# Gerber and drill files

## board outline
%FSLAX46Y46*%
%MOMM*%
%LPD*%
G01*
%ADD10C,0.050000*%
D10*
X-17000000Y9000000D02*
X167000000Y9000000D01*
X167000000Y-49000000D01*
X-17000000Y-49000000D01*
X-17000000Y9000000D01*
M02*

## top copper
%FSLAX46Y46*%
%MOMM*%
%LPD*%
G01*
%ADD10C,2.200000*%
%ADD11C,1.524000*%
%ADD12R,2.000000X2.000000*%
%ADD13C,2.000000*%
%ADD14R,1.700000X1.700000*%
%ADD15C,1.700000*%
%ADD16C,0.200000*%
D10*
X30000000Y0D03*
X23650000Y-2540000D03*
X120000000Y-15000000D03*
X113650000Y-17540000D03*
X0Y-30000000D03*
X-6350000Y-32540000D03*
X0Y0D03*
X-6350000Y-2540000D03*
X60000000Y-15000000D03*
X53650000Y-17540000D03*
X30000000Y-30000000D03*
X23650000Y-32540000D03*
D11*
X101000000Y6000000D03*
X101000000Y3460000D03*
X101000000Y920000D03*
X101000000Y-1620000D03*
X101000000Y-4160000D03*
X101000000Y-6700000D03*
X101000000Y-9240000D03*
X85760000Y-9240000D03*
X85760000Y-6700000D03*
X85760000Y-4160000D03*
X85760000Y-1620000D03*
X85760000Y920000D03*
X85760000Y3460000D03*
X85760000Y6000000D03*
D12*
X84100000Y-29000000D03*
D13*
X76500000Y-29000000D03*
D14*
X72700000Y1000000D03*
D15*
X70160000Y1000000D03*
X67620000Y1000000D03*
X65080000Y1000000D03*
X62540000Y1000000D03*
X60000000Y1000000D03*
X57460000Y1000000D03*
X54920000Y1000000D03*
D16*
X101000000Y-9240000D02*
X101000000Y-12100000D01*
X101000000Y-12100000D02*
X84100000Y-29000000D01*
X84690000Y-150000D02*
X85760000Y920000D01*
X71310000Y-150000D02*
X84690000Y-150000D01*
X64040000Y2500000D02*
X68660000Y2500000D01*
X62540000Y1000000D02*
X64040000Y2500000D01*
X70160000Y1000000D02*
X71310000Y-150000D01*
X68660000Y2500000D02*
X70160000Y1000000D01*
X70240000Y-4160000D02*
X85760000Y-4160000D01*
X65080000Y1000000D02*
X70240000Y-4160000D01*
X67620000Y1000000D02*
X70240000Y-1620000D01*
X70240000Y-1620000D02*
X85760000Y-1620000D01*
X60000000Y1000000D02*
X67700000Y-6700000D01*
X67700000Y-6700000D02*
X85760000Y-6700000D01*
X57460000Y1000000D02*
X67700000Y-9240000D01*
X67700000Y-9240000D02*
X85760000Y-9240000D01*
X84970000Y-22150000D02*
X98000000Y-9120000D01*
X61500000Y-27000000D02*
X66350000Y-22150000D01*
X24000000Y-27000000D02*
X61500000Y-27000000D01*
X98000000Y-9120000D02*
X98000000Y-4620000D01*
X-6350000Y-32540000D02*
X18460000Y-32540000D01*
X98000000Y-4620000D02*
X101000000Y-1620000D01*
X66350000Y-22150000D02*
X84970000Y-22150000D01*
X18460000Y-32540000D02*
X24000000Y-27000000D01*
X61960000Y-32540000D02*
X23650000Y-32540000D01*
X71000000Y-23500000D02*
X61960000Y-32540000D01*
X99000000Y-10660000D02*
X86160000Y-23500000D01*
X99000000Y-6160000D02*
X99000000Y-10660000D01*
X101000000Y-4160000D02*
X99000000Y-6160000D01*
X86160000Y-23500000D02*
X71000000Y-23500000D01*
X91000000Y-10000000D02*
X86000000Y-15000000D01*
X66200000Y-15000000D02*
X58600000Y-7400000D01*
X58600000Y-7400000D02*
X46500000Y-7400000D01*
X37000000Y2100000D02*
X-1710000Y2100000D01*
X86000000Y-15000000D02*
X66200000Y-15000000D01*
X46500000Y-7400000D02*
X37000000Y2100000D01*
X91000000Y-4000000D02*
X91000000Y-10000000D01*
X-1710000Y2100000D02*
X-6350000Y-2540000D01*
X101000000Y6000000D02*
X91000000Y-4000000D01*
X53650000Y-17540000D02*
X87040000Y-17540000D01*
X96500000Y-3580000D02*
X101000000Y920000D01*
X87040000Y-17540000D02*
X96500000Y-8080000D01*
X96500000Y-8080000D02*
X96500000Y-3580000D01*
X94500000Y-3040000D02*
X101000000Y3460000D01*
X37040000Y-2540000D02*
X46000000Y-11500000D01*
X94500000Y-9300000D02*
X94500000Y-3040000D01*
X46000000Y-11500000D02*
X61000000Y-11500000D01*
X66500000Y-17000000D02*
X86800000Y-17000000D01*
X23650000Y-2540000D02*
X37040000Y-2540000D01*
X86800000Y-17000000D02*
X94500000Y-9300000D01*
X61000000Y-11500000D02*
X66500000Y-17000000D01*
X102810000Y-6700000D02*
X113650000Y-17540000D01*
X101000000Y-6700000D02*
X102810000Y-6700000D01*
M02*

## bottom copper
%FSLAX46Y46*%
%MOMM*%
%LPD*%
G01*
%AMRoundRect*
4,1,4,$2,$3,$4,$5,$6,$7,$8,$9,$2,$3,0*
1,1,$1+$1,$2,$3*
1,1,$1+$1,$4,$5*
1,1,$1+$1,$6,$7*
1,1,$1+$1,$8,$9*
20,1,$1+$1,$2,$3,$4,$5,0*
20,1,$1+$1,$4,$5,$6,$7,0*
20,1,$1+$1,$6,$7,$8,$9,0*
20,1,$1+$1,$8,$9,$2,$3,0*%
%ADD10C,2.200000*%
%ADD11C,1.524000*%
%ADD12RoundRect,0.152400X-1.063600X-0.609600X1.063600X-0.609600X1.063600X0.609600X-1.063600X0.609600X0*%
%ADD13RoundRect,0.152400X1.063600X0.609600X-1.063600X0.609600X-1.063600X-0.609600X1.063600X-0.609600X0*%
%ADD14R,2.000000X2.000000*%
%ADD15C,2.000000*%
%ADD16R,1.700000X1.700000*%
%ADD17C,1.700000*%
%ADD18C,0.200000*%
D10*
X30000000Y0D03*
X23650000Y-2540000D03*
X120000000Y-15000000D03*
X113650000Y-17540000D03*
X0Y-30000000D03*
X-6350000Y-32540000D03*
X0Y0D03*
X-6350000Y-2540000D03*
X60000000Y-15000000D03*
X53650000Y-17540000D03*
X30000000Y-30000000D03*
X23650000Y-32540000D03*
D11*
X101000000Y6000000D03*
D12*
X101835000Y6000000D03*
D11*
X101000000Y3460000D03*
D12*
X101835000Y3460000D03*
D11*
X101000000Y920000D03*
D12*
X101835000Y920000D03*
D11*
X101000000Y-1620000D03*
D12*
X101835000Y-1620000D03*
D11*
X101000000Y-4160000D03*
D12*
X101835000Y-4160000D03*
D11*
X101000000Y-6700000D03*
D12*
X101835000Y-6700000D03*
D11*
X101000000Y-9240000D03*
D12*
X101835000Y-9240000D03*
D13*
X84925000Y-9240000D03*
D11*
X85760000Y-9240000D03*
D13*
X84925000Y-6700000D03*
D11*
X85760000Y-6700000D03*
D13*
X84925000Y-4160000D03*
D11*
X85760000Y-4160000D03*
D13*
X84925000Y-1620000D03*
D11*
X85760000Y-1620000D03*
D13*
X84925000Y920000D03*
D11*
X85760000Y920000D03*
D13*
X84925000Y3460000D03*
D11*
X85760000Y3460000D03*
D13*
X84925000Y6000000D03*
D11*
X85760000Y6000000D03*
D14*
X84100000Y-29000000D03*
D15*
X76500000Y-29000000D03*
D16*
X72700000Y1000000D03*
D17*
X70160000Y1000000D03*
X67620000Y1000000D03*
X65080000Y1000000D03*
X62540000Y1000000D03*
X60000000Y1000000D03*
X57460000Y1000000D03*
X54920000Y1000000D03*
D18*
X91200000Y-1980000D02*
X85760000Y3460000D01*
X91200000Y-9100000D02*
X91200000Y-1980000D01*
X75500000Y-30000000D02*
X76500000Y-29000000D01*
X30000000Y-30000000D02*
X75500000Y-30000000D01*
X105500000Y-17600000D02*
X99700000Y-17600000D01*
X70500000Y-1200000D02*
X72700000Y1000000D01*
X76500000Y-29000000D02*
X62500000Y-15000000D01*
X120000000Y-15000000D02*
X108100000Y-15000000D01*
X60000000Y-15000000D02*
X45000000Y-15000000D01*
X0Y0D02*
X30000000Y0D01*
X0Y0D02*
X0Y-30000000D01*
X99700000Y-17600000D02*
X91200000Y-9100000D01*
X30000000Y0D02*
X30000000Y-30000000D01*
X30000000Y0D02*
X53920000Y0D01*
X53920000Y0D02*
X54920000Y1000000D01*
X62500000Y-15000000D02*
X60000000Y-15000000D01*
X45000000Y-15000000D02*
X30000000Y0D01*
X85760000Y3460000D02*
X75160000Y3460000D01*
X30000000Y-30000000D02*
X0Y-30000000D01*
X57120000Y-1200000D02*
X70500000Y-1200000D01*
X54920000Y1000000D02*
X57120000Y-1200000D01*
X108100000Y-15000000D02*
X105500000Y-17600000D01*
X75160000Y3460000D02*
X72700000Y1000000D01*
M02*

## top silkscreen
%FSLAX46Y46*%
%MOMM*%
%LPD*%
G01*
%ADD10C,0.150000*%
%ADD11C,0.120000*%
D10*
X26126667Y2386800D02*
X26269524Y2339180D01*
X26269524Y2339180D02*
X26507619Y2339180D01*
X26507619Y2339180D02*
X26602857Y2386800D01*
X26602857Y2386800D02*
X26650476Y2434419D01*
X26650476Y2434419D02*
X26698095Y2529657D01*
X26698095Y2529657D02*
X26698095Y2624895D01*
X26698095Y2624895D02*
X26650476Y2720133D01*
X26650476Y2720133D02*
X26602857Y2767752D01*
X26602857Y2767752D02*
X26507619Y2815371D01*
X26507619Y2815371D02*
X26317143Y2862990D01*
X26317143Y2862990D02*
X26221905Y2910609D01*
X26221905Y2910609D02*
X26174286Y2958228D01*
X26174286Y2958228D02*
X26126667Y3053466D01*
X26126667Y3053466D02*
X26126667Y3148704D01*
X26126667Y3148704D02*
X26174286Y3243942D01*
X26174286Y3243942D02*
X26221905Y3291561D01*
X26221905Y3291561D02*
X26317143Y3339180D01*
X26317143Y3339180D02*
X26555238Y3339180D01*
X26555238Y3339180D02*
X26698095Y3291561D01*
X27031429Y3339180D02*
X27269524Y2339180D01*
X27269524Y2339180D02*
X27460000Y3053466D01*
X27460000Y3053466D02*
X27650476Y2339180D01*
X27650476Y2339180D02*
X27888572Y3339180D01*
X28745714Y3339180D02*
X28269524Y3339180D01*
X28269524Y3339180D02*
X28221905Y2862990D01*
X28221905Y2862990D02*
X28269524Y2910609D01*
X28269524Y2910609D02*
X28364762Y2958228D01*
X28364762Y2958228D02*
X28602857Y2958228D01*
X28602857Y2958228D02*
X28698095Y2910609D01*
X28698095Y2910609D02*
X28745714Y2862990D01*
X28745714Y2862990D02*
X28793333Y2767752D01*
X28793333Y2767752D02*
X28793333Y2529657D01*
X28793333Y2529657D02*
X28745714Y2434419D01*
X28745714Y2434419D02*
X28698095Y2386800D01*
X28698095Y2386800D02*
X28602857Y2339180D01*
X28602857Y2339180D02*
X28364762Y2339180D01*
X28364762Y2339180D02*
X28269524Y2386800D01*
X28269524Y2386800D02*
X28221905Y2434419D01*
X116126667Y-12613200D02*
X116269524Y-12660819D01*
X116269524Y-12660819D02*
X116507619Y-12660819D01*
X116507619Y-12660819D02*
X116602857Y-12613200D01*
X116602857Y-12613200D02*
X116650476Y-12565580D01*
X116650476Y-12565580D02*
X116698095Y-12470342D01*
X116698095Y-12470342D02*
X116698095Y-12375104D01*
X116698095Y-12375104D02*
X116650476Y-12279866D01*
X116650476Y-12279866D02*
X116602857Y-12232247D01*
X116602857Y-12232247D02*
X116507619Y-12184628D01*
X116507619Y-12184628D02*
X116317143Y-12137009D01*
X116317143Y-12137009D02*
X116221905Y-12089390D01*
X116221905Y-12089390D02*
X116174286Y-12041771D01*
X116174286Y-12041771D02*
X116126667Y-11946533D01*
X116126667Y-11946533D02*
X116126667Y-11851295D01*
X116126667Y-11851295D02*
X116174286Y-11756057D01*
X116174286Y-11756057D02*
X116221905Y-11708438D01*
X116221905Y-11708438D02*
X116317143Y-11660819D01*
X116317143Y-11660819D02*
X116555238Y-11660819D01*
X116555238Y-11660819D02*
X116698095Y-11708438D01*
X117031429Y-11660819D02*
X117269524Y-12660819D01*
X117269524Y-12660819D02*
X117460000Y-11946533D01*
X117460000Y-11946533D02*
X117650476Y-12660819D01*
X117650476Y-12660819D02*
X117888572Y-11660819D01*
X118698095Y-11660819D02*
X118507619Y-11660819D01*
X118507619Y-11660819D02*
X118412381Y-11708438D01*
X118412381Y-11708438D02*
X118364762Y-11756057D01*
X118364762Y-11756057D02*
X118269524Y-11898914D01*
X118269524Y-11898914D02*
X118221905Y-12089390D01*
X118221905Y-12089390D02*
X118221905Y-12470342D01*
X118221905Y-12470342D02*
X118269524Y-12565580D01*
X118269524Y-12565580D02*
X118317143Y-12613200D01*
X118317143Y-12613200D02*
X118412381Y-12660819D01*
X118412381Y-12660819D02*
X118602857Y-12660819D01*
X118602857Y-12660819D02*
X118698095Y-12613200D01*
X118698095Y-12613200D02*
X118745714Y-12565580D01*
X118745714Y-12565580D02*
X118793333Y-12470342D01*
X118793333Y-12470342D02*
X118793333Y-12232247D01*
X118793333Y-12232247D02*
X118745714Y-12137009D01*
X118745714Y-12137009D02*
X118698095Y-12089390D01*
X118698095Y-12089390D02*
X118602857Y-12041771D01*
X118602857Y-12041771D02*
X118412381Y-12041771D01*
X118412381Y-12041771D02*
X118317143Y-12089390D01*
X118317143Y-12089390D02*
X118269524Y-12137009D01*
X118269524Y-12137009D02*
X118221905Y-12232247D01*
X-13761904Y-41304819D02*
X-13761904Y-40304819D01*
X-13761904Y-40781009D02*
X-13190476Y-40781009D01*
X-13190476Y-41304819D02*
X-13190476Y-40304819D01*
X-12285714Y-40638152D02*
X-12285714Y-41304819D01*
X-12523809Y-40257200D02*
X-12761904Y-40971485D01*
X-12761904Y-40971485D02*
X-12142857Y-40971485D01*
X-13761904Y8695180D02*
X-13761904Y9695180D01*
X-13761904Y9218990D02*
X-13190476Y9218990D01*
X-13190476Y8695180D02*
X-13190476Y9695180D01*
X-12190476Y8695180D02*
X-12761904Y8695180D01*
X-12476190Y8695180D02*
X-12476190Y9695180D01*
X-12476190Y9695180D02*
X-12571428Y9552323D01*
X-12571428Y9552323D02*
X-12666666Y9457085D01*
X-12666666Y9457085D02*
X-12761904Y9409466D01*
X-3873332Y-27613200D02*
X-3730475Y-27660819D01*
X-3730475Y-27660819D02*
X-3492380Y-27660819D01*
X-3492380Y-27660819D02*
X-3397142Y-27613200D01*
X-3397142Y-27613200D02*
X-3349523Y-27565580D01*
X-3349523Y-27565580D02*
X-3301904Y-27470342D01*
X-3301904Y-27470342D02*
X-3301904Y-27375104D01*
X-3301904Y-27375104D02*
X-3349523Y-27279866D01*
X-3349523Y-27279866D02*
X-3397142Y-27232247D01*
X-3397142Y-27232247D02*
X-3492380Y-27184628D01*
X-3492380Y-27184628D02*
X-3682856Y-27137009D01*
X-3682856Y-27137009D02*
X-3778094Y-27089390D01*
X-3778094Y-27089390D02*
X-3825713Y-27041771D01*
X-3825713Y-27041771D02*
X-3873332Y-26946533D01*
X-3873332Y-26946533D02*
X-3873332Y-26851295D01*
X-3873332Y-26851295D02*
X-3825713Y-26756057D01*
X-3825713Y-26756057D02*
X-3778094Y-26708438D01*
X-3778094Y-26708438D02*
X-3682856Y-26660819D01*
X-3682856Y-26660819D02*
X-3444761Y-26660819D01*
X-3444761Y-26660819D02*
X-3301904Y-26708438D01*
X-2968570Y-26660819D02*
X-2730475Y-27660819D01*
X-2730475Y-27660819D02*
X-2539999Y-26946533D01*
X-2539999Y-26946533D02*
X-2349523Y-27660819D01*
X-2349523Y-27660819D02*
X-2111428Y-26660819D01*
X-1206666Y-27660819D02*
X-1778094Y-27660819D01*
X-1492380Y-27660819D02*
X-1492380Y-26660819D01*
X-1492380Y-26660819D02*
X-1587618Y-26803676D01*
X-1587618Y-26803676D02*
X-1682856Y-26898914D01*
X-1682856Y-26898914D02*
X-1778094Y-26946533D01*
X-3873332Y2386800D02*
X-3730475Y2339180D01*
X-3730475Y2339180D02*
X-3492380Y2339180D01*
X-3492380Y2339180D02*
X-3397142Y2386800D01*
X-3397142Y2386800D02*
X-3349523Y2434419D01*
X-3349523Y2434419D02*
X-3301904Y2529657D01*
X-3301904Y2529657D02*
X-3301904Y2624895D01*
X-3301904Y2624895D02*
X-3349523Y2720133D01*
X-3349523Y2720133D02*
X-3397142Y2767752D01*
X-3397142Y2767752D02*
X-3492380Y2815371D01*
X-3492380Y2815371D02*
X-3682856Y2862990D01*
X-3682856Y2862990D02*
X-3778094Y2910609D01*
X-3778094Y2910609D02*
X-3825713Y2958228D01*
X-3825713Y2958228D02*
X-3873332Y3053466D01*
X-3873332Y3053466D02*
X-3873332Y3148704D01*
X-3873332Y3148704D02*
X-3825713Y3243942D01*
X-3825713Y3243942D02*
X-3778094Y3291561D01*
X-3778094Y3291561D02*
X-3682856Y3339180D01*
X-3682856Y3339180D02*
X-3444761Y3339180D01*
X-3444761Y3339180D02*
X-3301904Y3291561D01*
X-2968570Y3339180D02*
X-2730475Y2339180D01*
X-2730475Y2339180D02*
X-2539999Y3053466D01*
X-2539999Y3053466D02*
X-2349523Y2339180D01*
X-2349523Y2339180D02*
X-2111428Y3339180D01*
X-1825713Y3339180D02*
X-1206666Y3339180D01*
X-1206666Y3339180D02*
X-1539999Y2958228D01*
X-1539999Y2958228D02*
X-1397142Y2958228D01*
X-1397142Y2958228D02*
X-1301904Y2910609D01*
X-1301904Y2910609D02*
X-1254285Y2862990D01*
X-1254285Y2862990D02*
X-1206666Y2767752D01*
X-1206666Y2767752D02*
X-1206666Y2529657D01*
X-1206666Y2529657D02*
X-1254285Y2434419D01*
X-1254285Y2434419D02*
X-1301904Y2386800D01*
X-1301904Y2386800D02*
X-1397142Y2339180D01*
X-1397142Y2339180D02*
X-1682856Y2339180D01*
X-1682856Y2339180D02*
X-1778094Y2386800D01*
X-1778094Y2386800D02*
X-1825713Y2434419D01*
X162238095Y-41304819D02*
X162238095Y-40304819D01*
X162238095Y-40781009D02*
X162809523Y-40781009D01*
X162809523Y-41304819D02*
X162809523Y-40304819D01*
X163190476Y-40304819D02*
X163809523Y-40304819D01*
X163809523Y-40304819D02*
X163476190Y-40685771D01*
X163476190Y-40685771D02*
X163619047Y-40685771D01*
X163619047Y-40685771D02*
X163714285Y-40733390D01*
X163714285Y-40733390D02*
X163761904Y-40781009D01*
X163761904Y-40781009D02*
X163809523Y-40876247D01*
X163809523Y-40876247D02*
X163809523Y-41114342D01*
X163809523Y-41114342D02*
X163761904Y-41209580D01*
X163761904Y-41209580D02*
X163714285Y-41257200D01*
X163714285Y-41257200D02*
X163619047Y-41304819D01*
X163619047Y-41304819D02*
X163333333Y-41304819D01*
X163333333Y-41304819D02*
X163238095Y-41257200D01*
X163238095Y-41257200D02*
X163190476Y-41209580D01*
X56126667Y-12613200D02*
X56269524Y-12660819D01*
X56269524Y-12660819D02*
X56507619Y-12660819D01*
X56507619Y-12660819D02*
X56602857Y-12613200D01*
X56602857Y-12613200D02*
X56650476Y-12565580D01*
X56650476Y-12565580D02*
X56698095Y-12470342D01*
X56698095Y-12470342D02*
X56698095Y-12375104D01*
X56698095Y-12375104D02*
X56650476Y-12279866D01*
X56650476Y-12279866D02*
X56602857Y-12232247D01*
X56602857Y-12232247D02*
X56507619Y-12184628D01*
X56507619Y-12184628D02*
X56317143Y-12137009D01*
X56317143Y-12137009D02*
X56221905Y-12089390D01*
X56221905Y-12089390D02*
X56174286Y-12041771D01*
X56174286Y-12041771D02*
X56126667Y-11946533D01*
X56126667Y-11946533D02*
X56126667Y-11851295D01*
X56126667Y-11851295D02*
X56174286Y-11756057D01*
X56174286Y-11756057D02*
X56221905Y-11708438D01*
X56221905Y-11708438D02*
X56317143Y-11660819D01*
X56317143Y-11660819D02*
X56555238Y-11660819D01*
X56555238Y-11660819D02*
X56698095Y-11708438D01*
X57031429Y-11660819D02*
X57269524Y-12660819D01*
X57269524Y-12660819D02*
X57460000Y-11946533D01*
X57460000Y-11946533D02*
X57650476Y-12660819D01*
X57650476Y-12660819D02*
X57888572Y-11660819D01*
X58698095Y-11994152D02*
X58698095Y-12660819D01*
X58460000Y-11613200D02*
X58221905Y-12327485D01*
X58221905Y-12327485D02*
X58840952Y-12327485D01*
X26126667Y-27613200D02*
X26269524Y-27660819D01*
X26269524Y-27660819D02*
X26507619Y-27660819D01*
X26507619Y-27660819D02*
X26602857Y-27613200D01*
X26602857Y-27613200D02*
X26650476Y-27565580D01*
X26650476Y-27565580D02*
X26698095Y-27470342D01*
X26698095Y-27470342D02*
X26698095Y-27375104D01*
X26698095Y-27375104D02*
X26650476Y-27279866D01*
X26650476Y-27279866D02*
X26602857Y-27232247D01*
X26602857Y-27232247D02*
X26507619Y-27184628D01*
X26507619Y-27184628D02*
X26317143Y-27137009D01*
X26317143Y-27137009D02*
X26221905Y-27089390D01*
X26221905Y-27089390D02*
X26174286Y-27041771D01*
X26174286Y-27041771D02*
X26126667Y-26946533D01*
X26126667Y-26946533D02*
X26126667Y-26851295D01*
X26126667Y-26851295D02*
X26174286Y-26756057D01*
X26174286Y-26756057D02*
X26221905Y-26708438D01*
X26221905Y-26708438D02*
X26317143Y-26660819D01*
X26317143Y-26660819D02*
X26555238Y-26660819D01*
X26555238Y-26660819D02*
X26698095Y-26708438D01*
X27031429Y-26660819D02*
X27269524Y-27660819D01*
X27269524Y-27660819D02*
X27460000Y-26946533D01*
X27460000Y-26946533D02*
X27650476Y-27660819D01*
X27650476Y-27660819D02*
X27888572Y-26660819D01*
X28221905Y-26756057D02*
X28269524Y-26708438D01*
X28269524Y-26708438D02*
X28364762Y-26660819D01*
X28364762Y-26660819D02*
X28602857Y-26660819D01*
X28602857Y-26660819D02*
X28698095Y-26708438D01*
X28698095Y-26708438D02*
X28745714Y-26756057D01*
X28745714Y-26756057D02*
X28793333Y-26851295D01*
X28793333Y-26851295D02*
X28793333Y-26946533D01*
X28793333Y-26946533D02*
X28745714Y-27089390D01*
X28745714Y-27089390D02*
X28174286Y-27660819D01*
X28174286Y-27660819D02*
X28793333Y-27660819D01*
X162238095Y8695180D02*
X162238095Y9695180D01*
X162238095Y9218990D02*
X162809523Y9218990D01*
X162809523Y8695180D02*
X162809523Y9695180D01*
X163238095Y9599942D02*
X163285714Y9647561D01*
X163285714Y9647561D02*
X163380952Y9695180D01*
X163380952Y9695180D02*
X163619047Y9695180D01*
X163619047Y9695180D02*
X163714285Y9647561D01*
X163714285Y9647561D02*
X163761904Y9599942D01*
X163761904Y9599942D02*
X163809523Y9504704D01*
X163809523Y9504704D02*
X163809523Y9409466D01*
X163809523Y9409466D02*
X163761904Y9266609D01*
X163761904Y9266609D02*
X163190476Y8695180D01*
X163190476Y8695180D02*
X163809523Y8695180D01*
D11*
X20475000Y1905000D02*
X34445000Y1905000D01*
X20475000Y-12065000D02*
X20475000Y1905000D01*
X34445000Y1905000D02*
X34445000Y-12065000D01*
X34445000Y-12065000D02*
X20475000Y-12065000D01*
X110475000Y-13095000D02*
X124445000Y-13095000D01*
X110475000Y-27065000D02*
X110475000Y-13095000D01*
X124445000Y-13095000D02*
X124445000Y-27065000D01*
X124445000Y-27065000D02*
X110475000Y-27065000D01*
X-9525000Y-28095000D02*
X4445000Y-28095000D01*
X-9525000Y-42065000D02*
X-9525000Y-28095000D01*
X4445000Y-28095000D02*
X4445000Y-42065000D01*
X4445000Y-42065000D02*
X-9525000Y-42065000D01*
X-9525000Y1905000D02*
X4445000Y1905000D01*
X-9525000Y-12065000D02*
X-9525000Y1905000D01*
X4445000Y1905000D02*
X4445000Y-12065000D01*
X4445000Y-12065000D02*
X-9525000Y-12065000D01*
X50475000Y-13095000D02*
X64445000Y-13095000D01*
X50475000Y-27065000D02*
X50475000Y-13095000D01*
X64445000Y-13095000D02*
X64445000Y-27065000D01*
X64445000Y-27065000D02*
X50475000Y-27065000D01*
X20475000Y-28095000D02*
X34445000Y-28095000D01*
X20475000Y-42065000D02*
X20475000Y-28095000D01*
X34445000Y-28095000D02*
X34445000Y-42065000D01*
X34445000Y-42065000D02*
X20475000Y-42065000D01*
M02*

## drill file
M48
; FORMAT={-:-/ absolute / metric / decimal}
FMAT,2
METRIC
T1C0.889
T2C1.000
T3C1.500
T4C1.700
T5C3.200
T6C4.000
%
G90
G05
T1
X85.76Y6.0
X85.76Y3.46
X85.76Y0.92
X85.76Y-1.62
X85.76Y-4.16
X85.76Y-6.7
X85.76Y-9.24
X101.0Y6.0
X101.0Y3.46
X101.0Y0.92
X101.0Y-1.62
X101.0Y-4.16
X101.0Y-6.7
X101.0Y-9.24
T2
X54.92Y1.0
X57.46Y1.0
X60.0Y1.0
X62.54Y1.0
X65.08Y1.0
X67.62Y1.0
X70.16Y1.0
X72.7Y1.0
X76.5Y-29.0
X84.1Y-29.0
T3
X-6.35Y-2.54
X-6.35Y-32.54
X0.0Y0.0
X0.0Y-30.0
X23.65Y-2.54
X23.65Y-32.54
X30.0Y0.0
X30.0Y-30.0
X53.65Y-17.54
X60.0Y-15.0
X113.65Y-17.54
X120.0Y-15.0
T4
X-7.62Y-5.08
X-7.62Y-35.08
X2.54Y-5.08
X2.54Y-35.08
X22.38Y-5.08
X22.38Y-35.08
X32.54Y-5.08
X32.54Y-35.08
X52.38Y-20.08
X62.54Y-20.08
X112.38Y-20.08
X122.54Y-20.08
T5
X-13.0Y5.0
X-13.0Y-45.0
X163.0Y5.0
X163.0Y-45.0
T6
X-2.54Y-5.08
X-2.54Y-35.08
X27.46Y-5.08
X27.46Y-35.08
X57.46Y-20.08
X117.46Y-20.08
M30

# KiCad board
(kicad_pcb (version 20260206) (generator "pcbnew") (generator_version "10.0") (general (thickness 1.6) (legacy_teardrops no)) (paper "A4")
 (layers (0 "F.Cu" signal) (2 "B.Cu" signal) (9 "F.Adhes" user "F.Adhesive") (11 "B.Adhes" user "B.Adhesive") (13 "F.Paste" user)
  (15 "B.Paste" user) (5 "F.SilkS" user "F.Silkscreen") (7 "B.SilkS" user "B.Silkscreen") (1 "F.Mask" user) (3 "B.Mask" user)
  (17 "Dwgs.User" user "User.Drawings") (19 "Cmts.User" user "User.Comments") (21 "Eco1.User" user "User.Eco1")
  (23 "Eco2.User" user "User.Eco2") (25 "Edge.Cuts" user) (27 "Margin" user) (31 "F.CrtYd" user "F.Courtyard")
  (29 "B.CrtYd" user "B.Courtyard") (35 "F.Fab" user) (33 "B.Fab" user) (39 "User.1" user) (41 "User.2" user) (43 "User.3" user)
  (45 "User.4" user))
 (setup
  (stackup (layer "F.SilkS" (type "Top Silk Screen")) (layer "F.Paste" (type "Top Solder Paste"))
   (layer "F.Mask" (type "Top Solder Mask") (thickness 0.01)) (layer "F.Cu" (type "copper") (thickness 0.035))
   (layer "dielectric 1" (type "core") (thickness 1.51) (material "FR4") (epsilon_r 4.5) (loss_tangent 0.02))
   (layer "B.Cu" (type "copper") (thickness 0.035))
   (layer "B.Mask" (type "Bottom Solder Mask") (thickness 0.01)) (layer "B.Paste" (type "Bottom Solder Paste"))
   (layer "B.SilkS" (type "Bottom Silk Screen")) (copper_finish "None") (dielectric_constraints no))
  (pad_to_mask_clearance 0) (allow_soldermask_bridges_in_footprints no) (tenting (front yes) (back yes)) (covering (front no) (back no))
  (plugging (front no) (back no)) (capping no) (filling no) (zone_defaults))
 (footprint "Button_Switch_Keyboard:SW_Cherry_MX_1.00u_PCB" (layer "F.Cu") (at 30 0)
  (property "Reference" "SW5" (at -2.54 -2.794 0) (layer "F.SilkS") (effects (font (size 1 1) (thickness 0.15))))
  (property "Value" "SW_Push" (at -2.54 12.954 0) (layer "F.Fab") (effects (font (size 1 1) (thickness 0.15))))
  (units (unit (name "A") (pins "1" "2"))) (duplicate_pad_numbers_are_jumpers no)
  (fp_line (start -9.525 -1.905) (end 4.445 -1.905) (stroke (width 0.12) (type solid)) (layer "F.SilkS"))
  (fp_line (start -9.525 12.065) (end -9.525 -1.905) (stroke (width 0.12) (type solid)) (layer "F.SilkS"))
  (fp_line (start 4.445 -1.905) (end 4.445 12.065) (stroke (width 0.12) (type solid)) (layer "F.SilkS"))
  (fp_line (start 4.445 12.065) (end -9.525 12.065) (stroke (width 0.12) (type solid)) (layer "F.SilkS"))
  (pad "" np_thru_hole circle (at -7.62 5.08) (size 1.7 1.7) (drill 1.7) (layers "*.Cu" "*.Mask"))
  (pad "" np_thru_hole circle (at -2.54 5.08) (size 4 4) (drill 4) (layers "*.Cu" "*.Mask"))
  (pad "" np_thru_hole circle (at 2.54 5.08) (size 1.7 1.7) (drill 1.7) (layers "*.Cu" "*.Mask"))
  (pad "1" thru_hole circle (at 0 0) (size 2.2 2.2) (drill 1.5) (layers "*.Cu" "*.Mask") (remove_unused_layers no) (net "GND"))
  (pad "2" thru_hole circle (at -6.35 2.54) (size 2.2 2.2) (drill 1.5) (layers "*.Cu" "*.Mask") (remove_unused_layers no) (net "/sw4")))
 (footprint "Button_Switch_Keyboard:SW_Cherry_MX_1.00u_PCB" (layer "F.Cu") (at 120 15)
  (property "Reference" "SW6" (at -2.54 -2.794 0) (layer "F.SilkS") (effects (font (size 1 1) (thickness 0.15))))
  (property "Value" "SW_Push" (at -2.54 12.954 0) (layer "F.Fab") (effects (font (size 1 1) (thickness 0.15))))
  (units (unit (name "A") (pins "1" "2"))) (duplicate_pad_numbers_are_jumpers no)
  (fp_line (start -9.525 -1.905) (end 4.445 -1.905) (stroke (width 0.12) (type solid)) (layer "F.SilkS"))
  (fp_line (start -9.525 12.065) (end -9.525 -1.905) (stroke (width 0.12) (type solid)) (layer "F.SilkS"))
  (fp_line (start 4.445 -1.905) (end 4.445 12.065) (stroke (width 0.12) (type solid)) (layer "F.SilkS"))
  (fp_line (start 4.445 12.065) (end -9.525 12.065) (stroke (width 0.12) (type solid)) (layer "F.SilkS"))
  (pad "" np_thru_hole circle (at -7.62 5.08) (size 1.7 1.7) (drill 1.7) (layers "*.Cu" "*.Mask"))
  (pad "" np_thru_hole circle (at -2.54 5.08) (size 4 4) (drill 4) (layers "*.Cu" "*.Mask"))
  (pad "" np_thru_hole circle (at 2.54 5.08) (size 1.7 1.7) (drill 1.7) (layers "*.Cu" "*.Mask"))
  (pad "1" thru_hole circle (at 0 0) (size 2.2 2.2) (drill 1.5) (layers "*.Cu" "*.Mask") (remove_unused_layers no) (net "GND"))
  (pad "2" thru_hole circle (at -6.35 2.54) (size 2.2 2.2) (drill 1.5) (layers "*.Cu" "*.Mask") (remove_unused_layers no) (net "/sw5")))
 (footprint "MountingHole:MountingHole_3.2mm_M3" (layer "F.Cu") (at -13 45)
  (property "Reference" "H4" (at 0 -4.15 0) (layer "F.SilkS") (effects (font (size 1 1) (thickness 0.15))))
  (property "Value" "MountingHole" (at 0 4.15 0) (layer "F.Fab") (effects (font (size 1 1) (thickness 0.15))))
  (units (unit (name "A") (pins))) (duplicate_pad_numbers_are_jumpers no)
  (pad "" np_thru_hole circle (at 0 0) (size 3.2 3.2) (drill 3.2) (layers "*.Cu" "*.Mask")))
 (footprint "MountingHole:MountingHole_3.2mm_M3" (layer "F.Cu") (at -13 -5)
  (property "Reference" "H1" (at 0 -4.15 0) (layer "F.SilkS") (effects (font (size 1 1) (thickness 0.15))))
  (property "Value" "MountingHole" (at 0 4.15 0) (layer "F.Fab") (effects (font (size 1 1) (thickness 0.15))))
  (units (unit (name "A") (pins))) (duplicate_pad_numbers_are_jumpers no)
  (pad "" np_thru_hole circle (at 0 0) (size 3.2 3.2) (drill 3.2) (layers "*.Cu" "*.Mask")))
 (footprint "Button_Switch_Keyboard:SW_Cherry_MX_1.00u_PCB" (layer "F.Cu") (at 0 30)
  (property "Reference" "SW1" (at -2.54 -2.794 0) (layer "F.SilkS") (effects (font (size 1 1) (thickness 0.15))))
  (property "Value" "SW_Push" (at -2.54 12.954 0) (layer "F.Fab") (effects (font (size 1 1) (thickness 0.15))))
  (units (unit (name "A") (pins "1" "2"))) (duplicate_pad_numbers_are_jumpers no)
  (fp_line (start -9.525 -1.905) (end 4.445 -1.905) (stroke (width 0.12) (type solid)) (layer "F.SilkS"))
  (fp_line (start -9.525 12.065) (end -9.525 -1.905) (stroke (width 0.12) (type solid)) (layer "F.SilkS"))
  (fp_line (start 4.445 -1.905) (end 4.445 12.065) (stroke (width 0.12) (type solid)) (layer "F.SilkS"))
  (fp_line (start 4.445 12.065) (end -9.525 12.065) (stroke (width 0.12) (type solid)) (layer "F.SilkS"))
  (pad "" np_thru_hole circle (at -7.62 5.08) (size 1.7 1.7) (drill 1.7) (layers "*.Cu" "*.Mask"))
  (pad "" np_thru_hole circle (at -2.54 5.08) (size 4 4) (drill 4) (layers "*.Cu" "*.Mask"))
  (pad "" np_thru_hole circle (at 2.54 5.08) (size 1.7 1.7) (drill 1.7) (layers "*.Cu" "*.Mask"))
  (pad "1" thru_hole circle (at 0 0) (size 2.2 2.2) (drill 1.5) (layers "*.Cu" "*.Mask") (remove_unused_layers no) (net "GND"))
  (pad "2" thru_hole circle (at -6.35 2.54) (size 2.2 2.2) (drill 1.5) (layers "*.Cu" "*.Mask") (remove_unused_layers no) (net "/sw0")))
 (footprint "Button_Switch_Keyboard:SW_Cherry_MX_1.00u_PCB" (layer "F.Cu") (at 0 0)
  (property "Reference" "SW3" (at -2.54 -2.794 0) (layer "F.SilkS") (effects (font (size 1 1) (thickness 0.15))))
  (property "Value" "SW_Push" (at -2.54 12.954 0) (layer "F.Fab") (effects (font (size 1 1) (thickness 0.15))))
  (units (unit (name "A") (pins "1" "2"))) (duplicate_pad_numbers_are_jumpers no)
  (fp_line (start -9.525 -1.905) (end 4.445 -1.905) (stroke (width 0.12) (type solid)) (layer "F.SilkS"))
  (fp_line (start -9.525 12.065) (end -9.525 -1.905) (stroke (width 0.12) (type solid)) (layer "F.SilkS"))
  (fp_line (start 4.445 -1.905) (end 4.445 12.065) (stroke (width 0.12) (type solid)) (layer "F.SilkS"))
  (fp_line (start 4.445 12.065) (end -9.525 12.065) (stroke (width 0.12) (type solid)) (layer "F.SilkS"))
  (pad "" np_thru_hole circle (at -7.62 5.08) (size 1.7 1.7) (drill 1.7) (layers "*.Cu" "*.Mask"))
  (pad "" np_thru_hole circle (at -2.54 5.08) (size 4 4) (drill 4) (layers "*.Cu" "*.Mask"))
  (pad "" np_thru_hole circle (at 2.54 5.08) (size 1.7 1.7) (drill 1.7) (layers "*.Cu" "*.Mask"))
  (pad "1" thru_hole circle (at 0 0) (size 2.2 2.2) (drill 1.5) (layers "*.Cu" "*.Mask") (remove_unused_layers no) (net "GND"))
  (pad "2" thru_hole circle (at -6.35 2.54) (size 2.2 2.2) (drill 1.5) (layers "*.Cu" "*.Mask") (remove_unused_layers no) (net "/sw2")))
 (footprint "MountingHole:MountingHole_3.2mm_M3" (layer "F.Cu") (at 163 45)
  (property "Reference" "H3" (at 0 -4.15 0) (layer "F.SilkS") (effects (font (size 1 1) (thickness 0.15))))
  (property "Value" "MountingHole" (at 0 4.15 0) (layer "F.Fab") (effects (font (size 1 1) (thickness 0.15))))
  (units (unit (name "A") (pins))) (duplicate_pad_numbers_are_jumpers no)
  (pad "" np_thru_hole circle (at 0 0) (size 3.2 3.2) (drill 3.2) (layers "*.Cu" "*.Mask")))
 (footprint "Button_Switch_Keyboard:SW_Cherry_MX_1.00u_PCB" (layer "F.Cu") (at 60 15)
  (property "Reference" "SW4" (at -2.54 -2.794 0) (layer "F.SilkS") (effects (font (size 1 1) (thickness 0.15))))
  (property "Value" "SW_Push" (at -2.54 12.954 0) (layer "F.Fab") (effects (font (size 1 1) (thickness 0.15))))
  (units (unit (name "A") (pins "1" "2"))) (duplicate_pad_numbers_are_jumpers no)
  (fp_line (start -9.525 -1.905) (end 4.445 -1.905) (stroke (width 0.12) (type solid)) (layer "F.SilkS"))
  (fp_line (start -9.525 12.065) (end -9.525 -1.905) (stroke (width 0.12) (type solid)) (layer "F.SilkS"))
  (fp_line (start 4.445 -1.905) (end 4.445 12.065) (stroke (width 0.12) (type solid)) (layer "F.SilkS"))
  (fp_line (start 4.445 12.065) (end -9.525 12.065) (stroke (width 0.12) (type solid)) (layer "F.SilkS"))
  (pad "" np_thru_hole circle (at -7.62 5.08) (size 1.7 1.7) (drill 1.7) (layers "*.Cu" "*.Mask"))
  (pad "" np_thru_hole circle (at -2.54 5.08) (size 4 4) (drill 4) (layers "*.Cu" "*.Mask"))
  (pad "" np_thru_hole circle (at 2.54 5.08) (size 1.7 1.7) (drill 1.7) (layers "*.Cu" "*.Mask"))
  (pad "1" thru_hole circle (at 0 0) (size 2.2 2.2) (drill 1.5) (layers "*.Cu" "*.Mask") (remove_unused_layers no) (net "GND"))
  (pad "2" thru_hole circle (at -6.35 2.54) (size 2.2 2.2) (drill 1.5) (layers "*.Cu" "*.Mask") (remove_unused_layers no) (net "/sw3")))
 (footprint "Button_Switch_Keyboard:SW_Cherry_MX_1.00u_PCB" (layer "F.Cu") (at 30 30)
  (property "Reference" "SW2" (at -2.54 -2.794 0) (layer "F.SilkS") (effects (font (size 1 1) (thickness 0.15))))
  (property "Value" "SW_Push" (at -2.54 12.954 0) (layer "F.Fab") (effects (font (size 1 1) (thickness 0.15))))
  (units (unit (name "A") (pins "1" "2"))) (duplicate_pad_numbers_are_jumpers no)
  (fp_line (start -9.525 -1.905) (end 4.445 -1.905) (stroke (width 0.12) (type solid)) (layer "F.SilkS"))
  (fp_line (start -9.525 12.065) (end -9.525 -1.905) (stroke (width 0.12) (type solid)) (layer "F.SilkS"))
  (fp_line (start 4.445 -1.905) (end 4.445 12.065) (stroke (width 0.12) (type solid)) (layer "F.SilkS"))
  (fp_line (start 4.445 12.065) (end -9.525 12.065) (stroke (width 0.12) (type solid)) (layer "F.SilkS"))
  (pad "" np_thru_hole circle (at -7.62 5.08) (size 1.7 1.7) (drill 1.7) (layers "*.Cu" "*.Mask"))
  (pad "" np_thru_hole circle (at -2.54 5.08) (size 4 4) (drill 4) (layers "*.Cu" "*.Mask"))
  (pad "" np_thru_hole circle (at 2.54 5.08) (size 1.7 1.7) (drill 1.7) (layers "*.Cu" "*.Mask"))
  (pad "1" thru_hole circle (at 0 0) (size 2.2 2.2) (drill 1.5) (layers "*.Cu" "*.Mask") (remove_unused_layers no) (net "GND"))
  (pad "2" thru_hole circle (at -6.35 2.54) (size 2.2 2.2) (drill 1.5) (layers "*.Cu" "*.Mask") (remove_unused_layers no) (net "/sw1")))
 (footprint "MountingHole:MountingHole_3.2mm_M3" (layer "F.Cu") (at 163 -5)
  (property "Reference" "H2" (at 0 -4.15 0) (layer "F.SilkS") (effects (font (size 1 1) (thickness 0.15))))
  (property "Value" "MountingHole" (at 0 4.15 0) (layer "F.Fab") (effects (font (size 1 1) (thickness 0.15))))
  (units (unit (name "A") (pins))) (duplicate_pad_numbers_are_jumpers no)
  (pad "" np_thru_hole circle (at 0 0) (size 3.2 3.2) (drill 3.2) (layers "*.Cu" "*.Mask")))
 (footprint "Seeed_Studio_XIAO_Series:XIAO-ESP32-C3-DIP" (layer "B.Cu") (at 93.38 1.62 90)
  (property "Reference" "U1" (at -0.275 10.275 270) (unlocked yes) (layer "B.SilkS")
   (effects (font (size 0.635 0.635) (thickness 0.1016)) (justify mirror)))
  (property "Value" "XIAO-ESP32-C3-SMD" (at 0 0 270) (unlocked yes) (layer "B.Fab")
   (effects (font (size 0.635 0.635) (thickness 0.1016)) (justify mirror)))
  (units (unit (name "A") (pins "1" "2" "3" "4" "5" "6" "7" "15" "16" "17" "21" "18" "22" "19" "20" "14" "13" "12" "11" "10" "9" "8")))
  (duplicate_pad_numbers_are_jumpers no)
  (pad "1" thru_hole circle (at 7.62 7.62) (size 1.524 1.524) (drill 0.889) (layers "*.Cu" "*.Mask") (remove_unused_layers no) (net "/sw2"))
  (pad "1" smd roundrect (at 7.62 8.455) (size 2.432 1.524) (layers "B.Cu" "B.Mask") (roundrect_rratio 0.1) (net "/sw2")
   (thermal_bridge_angle 45))
  (pad "2" thru_hole circle (at 5.08 7.62) (size 1.524 1.524) (drill 0.889) (layers "*.Cu" "*.Mask") (remove_unused_layers no) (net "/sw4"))
  (pad "2" smd roundrect (at 5.08 8.455) (size 2.432 1.524) (layers "B.Cu" "B.Mask") (roundrect_rratio 0.1) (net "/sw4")
   (thermal_bridge_angle 45))
  (pad "3" thru_hole circle (at 2.54 7.62) (size 1.524 1.524) (drill 0.889) (layers "*.Cu" "*.Mask") (remove_unused_layers no) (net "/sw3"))
  (pad "3" smd roundrect (at 2.54 8.455) (size 2.432 1.524) (layers "B.Cu" "B.Mask") (roundrect_rratio 0.1) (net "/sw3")
   (thermal_bridge_angle 45))
  (pad "4" thru_hole circle (at 0 7.62) (size 1.524 1.524) (drill 0.889) (layers "*.Cu" "*.Mask") (remove_unused_layers no) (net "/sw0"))
  (pad "4" smd roundrect (at 0 8.455) (size 2.432 1.524) (layers "B.Cu" "B.Mask") (roundrect_rratio 0.1) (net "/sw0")
   (thermal_bridge_angle 45))
  (pad "5" thru_hole circle (at -2.54 7.62) (size 1.524 1.524) (drill 0.889) (layers "*.Cu" "*.Mask") (remove_unused_layers no) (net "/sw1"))
  (pad "5" smd roundrect (at -2.54 8.455) (size 2.432 1.524) (layers "B.Cu" "B.Mask") (roundrect_rratio 0.1) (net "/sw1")
   (thermal_bridge_angle 45))
  (pad "6" thru_hole circle (at -5.08 7.62) (size 1.524 1.524) (drill 0.889) (layers "*.Cu" "*.Mask") (remove_unused_layers no) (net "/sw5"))
  (pad "6" smd roundrect (at -5.08 8.455) (size 2.432 1.524) (layers "B.Cu" "B.Mask") (roundrect_rratio 0.1) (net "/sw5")
   (thermal_bridge_angle 45))
  (pad "7" thru_hole circle (at -7.62 7.62) (size 1.524 1.524) (drill 0.889) (layers "*.Cu" "*.Mask") (remove_unused_layers no)
   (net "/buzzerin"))
  (pad "7" smd roundrect (at -7.62 8.455) (size 2.432 1.524) (layers "B.Cu" "B.Mask") (roundrect_rratio 0.1) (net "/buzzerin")
   (thermal_bridge_angle 45))
  (pad "8" smd roundrect (at -7.62 -8.455 180) (size 2.432 1.524) (layers "B.Cu" "B.Mask") (roundrect_rratio 0.1) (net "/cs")
   (thermal_bridge_angle 45))
  (pad "8" thru_hole circle (at -7.62 -7.62 180) (size 1.524 1.524) (drill 0.889) (layers "*.Cu" "*.Mask") (remove_unused_layers no)
   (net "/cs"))
  (pad "9" smd roundrect (at -5.08 -8.455 180) (size 2.432 1.524) (layers "B.Cu" "B.Mask") (roundrect_rratio 0.1) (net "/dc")
   (thermal_bridge_angle 45))
  (pad "9" thru_hole circle (at -5.08 -7.62 180) (size 1.524 1.524) (drill 0.889) (layers "*.Cu" "*.Mask") (remove_unused_layers no)
   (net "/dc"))
  (pad "10" smd roundrect (at -2.54 -8.455 180) (size 2.432 1.524) (layers "B.Cu" "B.Mask") (roundrect_rratio 0.1) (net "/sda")
   (thermal_bridge_angle 45))
  (pad "10" thru_hole circle (at -2.54 -7.62 180) (size 1.524 1.524) (drill 0.889) (layers "*.Cu" "*.Mask") (remove_unused_layers no)
   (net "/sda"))
  (pad "11" smd roundrect (at 0 -8.455 180) (size 2.432 1.524) (layers "B.Cu" "B.Mask") (roundrect_rratio 0.1) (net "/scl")
   (thermal_bridge_angle 45))
  (pad "11" thru_hole circle (at 0 -7.62 180) (size 1.524 1.524) (drill 0.889) (layers "*.Cu" "*.Mask") (remove_unused_layers no)
   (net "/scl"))
  (pad "12" smd roundrect (at 2.54 -8.455 180) (size 2.432 1.524) (layers "B.Cu" "B.Mask") (roundrect_rratio 0.1) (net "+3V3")
   (thermal_bridge_angle 45))
  (pad "12" thru_hole circle (at 2.54 -7.62 180) (size 1.524 1.524) (drill 0.889) (layers "*.Cu" "*.Mask") (remove_unused_layers no)
   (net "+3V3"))
  (pad "13" smd roundrect (at 5.08 -8.455 180) (size 2.432 1.524) (layers "B.Cu" "B.Mask") (roundrect_rratio 0.1) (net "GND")
   (thermal_bridge_angle 45))
  (pad "13" thru_hole circle (at 5.08 -7.62 180) (size 1.524 1.524) (drill 0.889) (layers "*.Cu" "*.Mask") (remove_unused_layers no)
   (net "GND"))
  (pad "14" smd roundrect (at 7.62 -8.455 180) (size 2.432 1.524) (layers "B.Cu" "B.Mask") (roundrect_rratio 0.1)
   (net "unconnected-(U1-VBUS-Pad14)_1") (thermal_bridge_angle 45))
  (pad "14" thru_hole circle (at 7.62 -7.62 180) (size 1.524 1.524) (drill 0.889) (layers "*.Cu" "*.Mask") (remove_unused_layers no)
   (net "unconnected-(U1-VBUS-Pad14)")))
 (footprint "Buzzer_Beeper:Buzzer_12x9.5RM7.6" (layer "B.Cu") (at 84.1 29 180)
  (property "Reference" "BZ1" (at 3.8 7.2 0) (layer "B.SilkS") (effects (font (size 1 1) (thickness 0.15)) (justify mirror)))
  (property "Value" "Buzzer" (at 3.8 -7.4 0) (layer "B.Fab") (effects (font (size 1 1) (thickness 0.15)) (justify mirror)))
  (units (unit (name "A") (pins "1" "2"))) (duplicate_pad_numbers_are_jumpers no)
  (pad "1" thru_hole rect (at 0 0 180) (size 2 2) (drill 1) (layers "*.Cu" "*.Mask") (remove_unused_layers no) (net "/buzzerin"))
  (pad "2" thru_hole circle (at 7.6 0 180) (size 2 2) (drill 1) (layers "*.Cu" "*.Mask") (remove_unused_layers no) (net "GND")))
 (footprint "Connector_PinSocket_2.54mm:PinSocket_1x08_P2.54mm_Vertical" (layer "B.Cu") (at 72.7 -1 90)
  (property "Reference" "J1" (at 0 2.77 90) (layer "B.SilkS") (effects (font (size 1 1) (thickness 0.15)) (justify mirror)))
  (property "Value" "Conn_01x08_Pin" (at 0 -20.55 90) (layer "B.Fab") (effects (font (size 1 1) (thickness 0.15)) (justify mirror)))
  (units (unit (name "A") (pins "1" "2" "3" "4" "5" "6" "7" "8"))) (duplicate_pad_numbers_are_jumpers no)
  (pad "1" thru_hole rect (at 0 0 90) (size 1.7 1.7) (drill 1) (layers "*.Cu" "*.Mask") (remove_unused_layers no) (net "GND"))
  (pad "2" thru_hole circle (at 0 -2.54 90) (size 1.7 1.7) (drill 1) (layers "*.Cu" "*.Mask") (remove_unused_layers no) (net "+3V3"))
  (pad "3" thru_hole circle (at 0 -5.08 90) (size 1.7 1.7) (drill 1) (layers "*.Cu" "*.Mask") (remove_unused_layers no) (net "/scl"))
  (pad "4" thru_hole circle (at 0 -7.62 90) (size 1.7 1.7) (drill 1) (layers "*.Cu" "*.Mask") (remove_unused_layers no) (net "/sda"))
  (pad "5" thru_hole circle (at 0 -10.16 90) (size 1.7 1.7) (drill 1) (layers "*.Cu" "*.Mask") (remove_unused_layers no) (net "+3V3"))
  (pad "6" thru_hole circle (at 0 -12.7 90) (size 1.7 1.7) (drill 1) (layers "*.Cu" "*.Mask") (remove_unused_layers no) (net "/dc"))
  (pad "7" thru_hole circle (at 0 -15.24 90) (size 1.7 1.7) (drill 1) (layers "*.Cu" "*.Mask") (remove_unused_layers no) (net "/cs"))
  (pad "8" thru_hole circle (at 0 -17.78 90) (size 1.7 1.7) (drill 1) (layers "*.Cu" "*.Mask") (remove_unused_layers no) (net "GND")))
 (gr_rect (start -17 -9) (end 167 49) (stroke (width 0.05) (type default)) (fill no) (layer "Edge.Cuts"))
 (segment (start 91.2 1.98) (end 85.76 -3.46) (width 0.2) (layer "B.Cu") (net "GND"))
 (segment (start 91.2 9.1) (end 91.2 1.98) (width 0.2) (layer "B.Cu") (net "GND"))
 (segment (start 75.5 30) (end 76.5 29) (width 0.2) (layer "B.Cu") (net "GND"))
 (segment (start 30 30) (end 75.5 30) (width 0.2) (layer "B.Cu") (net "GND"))
 (segment (start 105.5 17.6) (end 99.7 17.6) (width 0.2) (layer "B.Cu") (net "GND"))
 (segment (start 70.5 1.2) (end 72.7 -1) (width 0.2) (layer "B.Cu") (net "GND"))
 (segment (start 76.5 29) (end 62.5 15) (width 0.2) (layer "B.Cu") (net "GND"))
 (segment (start 120 15) (end 108.1 15) (width 0.2) (layer "B.Cu") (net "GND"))
 (segment (start 60 15) (end 45 15) (width 0.2) (layer "B.Cu") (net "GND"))
 (segment (start 0 0) (end 30 0) (width 0.2) (layer "B.Cu") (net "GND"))
 (segment (start 0 0) (end 0 30) (width 0.2) (layer "B.Cu") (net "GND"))
 (segment (start 99.7 17.6) (end 91.2 9.1) (width 0.2) (layer "B.Cu") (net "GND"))
 (segment (start 30 0) (end 30 30) (width 0.2) (layer "B.Cu") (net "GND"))
 (segment (start 30 0) (end 53.92 0) (width 0.2) (layer "B.Cu") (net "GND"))
 (segment (start 53.92 0) (end 54.92 -1) (width 0.2) (layer "B.Cu") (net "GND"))
 (segment (start 62.5 15) (end 60 15) (width 0.2) (layer "B.Cu") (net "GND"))
 (segment (start 45 15) (end 30 0) (width 0.2) (layer "B.Cu") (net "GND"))
 (segment (start 85.76 -3.46) (end 75.16 -3.46) (width 0.2) (layer "B.Cu") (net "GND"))
 (segment (start 30 30) (end 0 30) (width 0.2) (layer "B.Cu") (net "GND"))
 (segment (start 57.12 1.2) (end 70.5 1.2) (width 0.2) (layer "B.Cu") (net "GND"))
 (segment (start 54.92 -1) (end 57.12 1.2) (width 0.2) (layer "B.Cu") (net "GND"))
 (segment (start 108.1 15) (end 105.5 17.6) (width 0.2) (layer "B.Cu") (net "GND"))
 (segment (start 75.16 -3.46) (end 72.7 -1) (width 0.2) (layer "B.Cu") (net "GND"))
 (segment (start 101 9.24) (end 101 12.1) (width 0.2) (layer "F.Cu") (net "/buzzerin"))
 (segment (start 101 12.1) (end 84.1 29) (width 0.2) (layer "F.Cu") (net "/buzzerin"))
 (segment (start 84.69 0.15) (end 85.76 -0.92) (width 0.2) (layer "F.Cu") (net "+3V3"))
 (segment (start 71.31 0.15) (end 84.69 0.15) (width 0.2) (layer "F.Cu") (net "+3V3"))
 (segment (start 64.04 -2.5) (end 68.66 -2.5) (width 0.2) (layer "F.Cu") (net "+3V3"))
 (segment (start 62.54 -1) (end 64.04 -2.5) (width 0.2) (layer "F.Cu") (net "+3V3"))
 (segment (start 70.16 -1) (end 71.31 0.15) (width 0.2) (layer "F.Cu") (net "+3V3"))
 (segment (start 68.66 -2.5) (end 70.16 -1) (width 0.2) (layer "F.Cu") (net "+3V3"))
 (segment (start 70.24 4.16) (end 85.76 4.16) (width 0.2) (layer "F.Cu") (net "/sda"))
 (segment (start 65.08 -1) (end 70.24 4.16) (width 0.2) (layer "F.Cu") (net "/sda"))
 (segment (start 67.62 -1) (end 70.24 1.62) (width 0.2) (layer "F.Cu") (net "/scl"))
 (segment (start 70.24 1.62) (end 85.76 1.62) (width 0.2) (layer "F.Cu") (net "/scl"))
 (segment (start 60 -1) (end 67.7 6.7) (width 0.2) (layer "F.Cu") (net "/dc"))
 (segment (start 67.7 6.7) (end 85.76 6.7) (width 0.2) (layer "F.Cu") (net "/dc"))
 (segment (start 57.46 -1) (end 67.7 9.24) (width 0.2) (layer "F.Cu") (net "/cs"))
 (segment (start 67.7 9.24) (end 85.76 9.24) (width 0.2) (layer "F.Cu") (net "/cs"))
 (segment (start 84.97 22.15) (end 98 9.12) (width 0.2) (layer "F.Cu") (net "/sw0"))
 (segment (start 61.5 27) (end 66.35 22.15) (width 0.2) (layer "F.Cu") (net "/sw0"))
 (segment (start 24 27) (end 61.5 27) (width 0.2) (layer "F.Cu") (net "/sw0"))
 (segment (start 98 9.12) (end 98 4.62) (width 0.2) (layer "F.Cu") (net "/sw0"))
 (segment (start -6.35 32.54) (end 18.46 32.54) (width 0.2) (layer "F.Cu") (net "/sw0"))
 (segment (start 98 4.62) (end 101 1.62) (width 0.2) (layer "F.Cu") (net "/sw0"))
 (segment (start 66.35 22.15) (end 84.97 22.15) (width 0.2) (layer "F.Cu") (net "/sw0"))
 (segment (start 18.46 32.54) (end 24 27) (width 0.2) (layer "F.Cu") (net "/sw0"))
 (segment (start 61.96 32.54) (end 23.65 32.54) (width 0.2) (layer "F.Cu") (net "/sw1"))
 (segment (start 71 23.5) (end 61.96 32.54) (width 0.2) (layer "F.Cu") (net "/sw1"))
 (segment (start 99 10.66) (end 86.16 23.5) (width 0.2) (layer "F.Cu") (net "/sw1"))
 (segment (start 99 6.16) (end 99 10.66) (width 0.2) (layer "F.Cu") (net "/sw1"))
 (segment (start 101 4.16) (end 99 6.16) (width 0.2) (layer "F.Cu") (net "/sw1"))
 (segment (start 86.16 23.5) (end 71 23.5) (width 0.2) (layer "F.Cu") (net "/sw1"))
 (segment (start 91 10) (end 86 15) (width 0.2) (layer "F.Cu") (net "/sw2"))
 (segment (start 66.2 15) (end 58.6 7.4) (width 0.2) (layer "F.Cu") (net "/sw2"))
 (segment (start 58.6 7.4) (end 46.5 7.4) (width 0.2) (layer "F.Cu") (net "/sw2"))
 (segment (start 37 -2.1) (end -1.71 -2.1) (width 0.2) (layer "F.Cu") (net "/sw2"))
 (segment (start 86 15) (end 66.2 15) (width 0.2) (layer "F.Cu") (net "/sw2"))
 (segment (start 46.5 7.4) (end 37 -2.1) (width 0.2) (layer "F.Cu") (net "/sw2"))
 (segment (start 91 4) (end 91 10) (width 0.2) (layer "F.Cu") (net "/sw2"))
 (segment (start -1.71 -2.1) (end -6.35 2.54) (width 0.2) (layer "F.Cu") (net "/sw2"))
 (segment (start 101 -6) (end 91 4) (width 0.2) (layer "F.Cu") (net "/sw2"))
 (segment (start 53.65 17.54) (end 87.04 17.54) (width 0.2) (layer "F.Cu") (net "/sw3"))
 (segment (start 96.5 3.58) (end 101 -0.92) (width 0.2) (layer "F.Cu") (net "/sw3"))
 (segment (start 87.04 17.54) (end 96.5 8.08) (width 0.2) (layer "F.Cu") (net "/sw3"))
 (segment (start 96.5 8.08) (end 96.5 3.58) (width 0.2) (layer "F.Cu") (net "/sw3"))
 (segment (start 94.5 3.04) (end 101 -3.46) (width 0.2) (layer "F.Cu") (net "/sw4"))
 (segment (start 37.04 2.54) (end 46 11.5) (width 0.2) (layer "F.Cu") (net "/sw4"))
 (segment (start 94.5 9.3) (end 94.5 3.04) (width 0.2) (layer "F.Cu") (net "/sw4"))
 (segment (start 46 11.5) (end 61 11.5) (width 0.2) (layer "F.Cu") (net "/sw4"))
 (segment (start 66.5 17) (end 86.8 17) (width 0.2) (layer "F.Cu") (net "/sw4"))
 (segment (start 23.65 2.54) (end 37.04 2.54) (width 0.2) (layer "F.Cu") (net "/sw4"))
 (segment (start 86.8 17) (end 94.5 9.3) (width 0.2) (layer "F.Cu") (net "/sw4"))
 (segment (start 61 11.5) (end 66.5 17) (width 0.2) (layer "F.Cu") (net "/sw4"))
 (segment (start 102.81 6.7) (end 113.65 17.54) (width 0.2) (layer "F.Cu") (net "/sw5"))
 (segment (start 101 6.7) (end 102.81 6.7) (width 0.2) (layer "F.Cu") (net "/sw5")))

